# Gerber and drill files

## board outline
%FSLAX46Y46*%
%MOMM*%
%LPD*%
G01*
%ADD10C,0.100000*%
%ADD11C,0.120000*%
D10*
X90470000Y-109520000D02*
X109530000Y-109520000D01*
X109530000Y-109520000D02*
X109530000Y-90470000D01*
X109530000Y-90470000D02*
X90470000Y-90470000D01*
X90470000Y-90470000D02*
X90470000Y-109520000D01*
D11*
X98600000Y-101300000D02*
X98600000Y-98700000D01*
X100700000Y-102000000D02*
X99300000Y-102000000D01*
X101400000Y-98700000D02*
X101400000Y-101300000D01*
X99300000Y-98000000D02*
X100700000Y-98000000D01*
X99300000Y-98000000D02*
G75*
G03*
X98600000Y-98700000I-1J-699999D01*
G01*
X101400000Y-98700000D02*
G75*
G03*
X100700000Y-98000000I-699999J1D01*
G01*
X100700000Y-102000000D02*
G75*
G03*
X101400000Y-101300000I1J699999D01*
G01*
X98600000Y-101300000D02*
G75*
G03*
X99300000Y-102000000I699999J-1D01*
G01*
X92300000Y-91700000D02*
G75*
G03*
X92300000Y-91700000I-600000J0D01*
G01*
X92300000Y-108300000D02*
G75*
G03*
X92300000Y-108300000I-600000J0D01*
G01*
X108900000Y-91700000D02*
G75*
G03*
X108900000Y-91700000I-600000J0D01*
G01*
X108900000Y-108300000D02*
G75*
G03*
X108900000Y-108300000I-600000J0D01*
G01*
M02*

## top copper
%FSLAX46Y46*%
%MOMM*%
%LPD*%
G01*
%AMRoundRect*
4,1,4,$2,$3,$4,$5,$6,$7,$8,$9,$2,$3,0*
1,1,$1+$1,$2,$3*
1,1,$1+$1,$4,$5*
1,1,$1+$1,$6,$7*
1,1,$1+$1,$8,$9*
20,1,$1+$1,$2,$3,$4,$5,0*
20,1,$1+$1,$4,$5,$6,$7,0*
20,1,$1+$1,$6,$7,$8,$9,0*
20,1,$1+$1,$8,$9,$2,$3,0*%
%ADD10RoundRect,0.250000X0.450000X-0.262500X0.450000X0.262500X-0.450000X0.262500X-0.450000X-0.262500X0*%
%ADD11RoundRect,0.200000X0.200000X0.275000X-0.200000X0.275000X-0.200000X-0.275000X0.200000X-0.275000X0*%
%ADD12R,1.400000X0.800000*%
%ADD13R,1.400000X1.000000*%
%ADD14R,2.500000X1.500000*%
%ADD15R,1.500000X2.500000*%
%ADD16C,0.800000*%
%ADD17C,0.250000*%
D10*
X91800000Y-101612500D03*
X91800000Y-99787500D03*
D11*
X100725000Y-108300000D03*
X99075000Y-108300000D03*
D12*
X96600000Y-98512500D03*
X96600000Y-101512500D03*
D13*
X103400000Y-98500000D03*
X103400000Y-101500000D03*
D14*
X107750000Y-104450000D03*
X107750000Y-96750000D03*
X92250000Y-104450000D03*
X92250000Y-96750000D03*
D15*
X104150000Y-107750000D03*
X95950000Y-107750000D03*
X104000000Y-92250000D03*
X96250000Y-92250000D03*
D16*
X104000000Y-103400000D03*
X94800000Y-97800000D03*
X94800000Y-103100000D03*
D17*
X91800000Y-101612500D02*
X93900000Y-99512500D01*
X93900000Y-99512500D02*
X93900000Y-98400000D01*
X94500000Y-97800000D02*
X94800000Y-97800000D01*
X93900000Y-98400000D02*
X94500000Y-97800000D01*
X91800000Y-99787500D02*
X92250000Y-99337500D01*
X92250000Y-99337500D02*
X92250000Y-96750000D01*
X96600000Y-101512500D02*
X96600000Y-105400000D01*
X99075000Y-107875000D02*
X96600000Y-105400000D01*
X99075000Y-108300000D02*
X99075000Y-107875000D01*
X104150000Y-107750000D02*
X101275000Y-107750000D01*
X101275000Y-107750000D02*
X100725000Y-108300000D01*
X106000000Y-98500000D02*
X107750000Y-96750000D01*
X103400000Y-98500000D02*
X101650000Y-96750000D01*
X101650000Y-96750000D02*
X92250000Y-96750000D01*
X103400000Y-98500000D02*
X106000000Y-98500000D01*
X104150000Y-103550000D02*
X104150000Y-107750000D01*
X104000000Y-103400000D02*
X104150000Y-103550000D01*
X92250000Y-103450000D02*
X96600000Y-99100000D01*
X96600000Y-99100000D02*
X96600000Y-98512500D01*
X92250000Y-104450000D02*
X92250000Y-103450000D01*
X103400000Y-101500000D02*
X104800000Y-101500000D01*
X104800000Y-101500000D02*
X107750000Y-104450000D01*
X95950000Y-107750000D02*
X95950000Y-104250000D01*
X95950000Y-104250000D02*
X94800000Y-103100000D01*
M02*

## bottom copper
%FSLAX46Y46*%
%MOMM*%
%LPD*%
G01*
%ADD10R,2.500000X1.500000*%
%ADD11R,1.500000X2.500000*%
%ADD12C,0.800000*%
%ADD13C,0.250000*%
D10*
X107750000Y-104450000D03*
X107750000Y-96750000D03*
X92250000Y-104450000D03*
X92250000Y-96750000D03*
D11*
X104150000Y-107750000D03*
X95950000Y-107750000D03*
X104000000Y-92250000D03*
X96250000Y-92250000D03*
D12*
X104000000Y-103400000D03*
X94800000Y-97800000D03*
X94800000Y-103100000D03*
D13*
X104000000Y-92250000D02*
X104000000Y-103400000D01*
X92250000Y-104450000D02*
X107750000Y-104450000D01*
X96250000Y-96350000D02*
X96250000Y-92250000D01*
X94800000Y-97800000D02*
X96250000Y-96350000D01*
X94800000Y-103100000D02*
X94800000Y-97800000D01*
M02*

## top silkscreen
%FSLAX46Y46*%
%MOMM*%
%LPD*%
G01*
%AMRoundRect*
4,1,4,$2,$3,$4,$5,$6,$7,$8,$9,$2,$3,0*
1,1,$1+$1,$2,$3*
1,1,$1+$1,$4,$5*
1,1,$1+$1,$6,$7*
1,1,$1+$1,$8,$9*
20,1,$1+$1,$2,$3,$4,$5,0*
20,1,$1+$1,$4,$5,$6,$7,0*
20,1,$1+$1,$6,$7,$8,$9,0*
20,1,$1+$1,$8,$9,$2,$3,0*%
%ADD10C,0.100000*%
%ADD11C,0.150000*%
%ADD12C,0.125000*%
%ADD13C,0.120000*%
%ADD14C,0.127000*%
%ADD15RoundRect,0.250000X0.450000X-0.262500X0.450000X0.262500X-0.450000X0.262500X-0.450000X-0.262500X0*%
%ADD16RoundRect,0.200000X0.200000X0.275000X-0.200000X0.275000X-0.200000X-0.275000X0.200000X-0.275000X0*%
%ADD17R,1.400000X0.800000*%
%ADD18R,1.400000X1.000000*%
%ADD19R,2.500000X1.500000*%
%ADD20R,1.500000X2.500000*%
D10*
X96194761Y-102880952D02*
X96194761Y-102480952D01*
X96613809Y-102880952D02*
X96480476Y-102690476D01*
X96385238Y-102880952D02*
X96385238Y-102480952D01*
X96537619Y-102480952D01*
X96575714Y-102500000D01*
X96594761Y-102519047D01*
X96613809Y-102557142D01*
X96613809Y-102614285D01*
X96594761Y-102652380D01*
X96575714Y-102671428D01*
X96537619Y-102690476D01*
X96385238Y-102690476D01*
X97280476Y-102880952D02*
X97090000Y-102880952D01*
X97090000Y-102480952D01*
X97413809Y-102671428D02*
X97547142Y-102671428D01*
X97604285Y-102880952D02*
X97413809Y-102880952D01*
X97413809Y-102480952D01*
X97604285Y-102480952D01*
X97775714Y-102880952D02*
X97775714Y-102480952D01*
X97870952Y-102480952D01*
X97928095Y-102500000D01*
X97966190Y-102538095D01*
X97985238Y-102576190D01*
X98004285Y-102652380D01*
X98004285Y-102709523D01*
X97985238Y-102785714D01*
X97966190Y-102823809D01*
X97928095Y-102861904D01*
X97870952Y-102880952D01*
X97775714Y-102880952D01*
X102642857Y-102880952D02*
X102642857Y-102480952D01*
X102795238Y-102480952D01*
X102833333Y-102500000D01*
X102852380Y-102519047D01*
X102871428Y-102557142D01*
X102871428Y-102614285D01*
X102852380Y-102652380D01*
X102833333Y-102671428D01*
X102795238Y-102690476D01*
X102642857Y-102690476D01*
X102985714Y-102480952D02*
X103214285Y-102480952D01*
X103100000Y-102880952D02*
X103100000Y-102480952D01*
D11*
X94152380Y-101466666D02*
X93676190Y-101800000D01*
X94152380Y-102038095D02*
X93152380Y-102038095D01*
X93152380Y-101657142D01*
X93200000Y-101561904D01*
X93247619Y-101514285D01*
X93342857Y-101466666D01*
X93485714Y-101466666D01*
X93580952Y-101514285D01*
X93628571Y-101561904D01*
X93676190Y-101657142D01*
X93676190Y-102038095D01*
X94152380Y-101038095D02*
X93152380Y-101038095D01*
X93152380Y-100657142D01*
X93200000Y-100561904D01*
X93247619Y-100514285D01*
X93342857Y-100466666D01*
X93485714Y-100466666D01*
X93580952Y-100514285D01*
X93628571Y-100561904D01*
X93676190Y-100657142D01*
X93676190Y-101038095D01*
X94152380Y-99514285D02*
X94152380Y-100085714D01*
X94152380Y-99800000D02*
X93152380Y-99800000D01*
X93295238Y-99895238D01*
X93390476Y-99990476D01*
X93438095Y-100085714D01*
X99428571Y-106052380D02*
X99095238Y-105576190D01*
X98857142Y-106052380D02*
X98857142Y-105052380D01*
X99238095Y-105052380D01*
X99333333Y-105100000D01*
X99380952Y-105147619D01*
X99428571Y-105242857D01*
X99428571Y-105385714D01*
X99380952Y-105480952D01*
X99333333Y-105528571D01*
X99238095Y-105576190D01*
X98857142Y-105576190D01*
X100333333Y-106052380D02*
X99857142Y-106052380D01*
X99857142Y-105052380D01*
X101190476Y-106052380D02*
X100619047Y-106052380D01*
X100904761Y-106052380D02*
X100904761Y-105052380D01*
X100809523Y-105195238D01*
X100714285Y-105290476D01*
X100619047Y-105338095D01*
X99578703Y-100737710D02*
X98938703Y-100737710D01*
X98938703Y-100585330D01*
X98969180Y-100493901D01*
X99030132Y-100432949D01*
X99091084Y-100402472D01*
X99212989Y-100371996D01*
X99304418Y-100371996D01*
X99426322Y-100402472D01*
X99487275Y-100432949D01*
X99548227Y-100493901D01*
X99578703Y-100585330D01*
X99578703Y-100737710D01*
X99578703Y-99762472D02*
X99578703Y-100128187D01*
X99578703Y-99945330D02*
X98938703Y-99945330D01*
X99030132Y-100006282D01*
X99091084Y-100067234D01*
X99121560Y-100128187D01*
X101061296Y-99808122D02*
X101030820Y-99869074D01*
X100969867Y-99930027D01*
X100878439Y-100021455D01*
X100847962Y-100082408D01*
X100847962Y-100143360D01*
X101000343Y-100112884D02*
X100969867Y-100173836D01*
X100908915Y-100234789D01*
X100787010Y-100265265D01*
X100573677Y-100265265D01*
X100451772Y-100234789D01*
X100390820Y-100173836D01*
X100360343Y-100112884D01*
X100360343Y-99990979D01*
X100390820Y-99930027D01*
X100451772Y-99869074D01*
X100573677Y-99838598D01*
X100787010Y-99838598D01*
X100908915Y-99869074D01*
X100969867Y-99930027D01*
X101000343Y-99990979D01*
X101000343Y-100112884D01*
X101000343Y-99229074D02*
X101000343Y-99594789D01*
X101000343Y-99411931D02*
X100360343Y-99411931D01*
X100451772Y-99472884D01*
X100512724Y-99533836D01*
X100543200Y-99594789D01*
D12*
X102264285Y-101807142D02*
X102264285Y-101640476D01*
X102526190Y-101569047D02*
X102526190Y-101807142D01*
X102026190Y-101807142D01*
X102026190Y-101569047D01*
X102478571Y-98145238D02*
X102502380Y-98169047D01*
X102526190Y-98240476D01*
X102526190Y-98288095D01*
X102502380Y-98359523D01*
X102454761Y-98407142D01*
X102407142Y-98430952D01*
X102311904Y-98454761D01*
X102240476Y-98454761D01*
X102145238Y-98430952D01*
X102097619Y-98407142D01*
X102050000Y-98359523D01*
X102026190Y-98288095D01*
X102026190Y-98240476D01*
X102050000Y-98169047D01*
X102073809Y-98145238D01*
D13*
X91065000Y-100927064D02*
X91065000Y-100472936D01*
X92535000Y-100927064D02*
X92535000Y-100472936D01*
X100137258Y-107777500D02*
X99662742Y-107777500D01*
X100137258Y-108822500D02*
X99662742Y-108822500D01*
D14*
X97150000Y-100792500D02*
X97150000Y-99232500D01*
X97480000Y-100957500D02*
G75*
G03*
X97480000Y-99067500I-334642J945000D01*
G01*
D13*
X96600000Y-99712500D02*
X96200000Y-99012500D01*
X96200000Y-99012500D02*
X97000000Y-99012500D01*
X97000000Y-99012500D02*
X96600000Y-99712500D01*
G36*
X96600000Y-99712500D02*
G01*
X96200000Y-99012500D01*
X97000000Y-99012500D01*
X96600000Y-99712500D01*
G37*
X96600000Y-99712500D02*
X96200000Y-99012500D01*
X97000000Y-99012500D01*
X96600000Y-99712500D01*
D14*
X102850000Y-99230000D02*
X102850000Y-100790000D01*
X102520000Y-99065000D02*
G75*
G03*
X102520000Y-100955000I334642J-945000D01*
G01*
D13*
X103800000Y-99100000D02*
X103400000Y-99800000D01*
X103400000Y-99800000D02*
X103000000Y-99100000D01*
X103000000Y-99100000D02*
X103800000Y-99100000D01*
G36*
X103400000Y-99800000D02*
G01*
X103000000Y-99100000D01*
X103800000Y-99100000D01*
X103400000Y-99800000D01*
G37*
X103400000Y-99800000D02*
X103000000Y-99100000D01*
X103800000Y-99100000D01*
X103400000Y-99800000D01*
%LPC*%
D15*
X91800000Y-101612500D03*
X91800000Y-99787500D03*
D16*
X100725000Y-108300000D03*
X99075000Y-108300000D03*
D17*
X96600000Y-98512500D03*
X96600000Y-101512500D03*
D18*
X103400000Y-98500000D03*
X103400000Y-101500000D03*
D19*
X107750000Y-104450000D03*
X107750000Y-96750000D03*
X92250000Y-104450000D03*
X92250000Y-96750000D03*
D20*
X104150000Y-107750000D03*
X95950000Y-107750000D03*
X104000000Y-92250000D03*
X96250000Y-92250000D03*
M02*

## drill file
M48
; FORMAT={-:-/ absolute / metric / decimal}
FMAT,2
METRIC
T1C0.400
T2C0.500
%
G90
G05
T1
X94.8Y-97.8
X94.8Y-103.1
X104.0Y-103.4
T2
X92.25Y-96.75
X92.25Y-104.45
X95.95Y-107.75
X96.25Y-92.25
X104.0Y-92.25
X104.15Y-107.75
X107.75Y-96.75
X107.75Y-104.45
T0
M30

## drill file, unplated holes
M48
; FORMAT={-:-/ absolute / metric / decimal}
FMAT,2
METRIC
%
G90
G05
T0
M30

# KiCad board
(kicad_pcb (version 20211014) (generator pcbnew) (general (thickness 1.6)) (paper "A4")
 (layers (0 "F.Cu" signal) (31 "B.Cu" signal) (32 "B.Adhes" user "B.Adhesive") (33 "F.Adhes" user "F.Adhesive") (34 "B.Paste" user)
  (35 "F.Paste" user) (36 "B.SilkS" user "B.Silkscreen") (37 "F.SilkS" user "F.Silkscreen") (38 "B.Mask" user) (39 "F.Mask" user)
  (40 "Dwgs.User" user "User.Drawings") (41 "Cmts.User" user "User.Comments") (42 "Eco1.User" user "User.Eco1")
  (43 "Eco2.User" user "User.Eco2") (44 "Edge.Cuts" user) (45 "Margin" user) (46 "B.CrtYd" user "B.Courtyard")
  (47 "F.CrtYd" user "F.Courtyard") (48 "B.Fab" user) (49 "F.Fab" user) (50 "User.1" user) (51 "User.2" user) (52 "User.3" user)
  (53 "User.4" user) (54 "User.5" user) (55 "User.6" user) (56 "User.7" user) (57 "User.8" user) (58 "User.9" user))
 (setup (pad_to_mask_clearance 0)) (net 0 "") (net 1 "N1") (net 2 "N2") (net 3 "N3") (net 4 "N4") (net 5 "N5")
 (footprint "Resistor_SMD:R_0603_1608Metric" (layer "F.Cu") (at 99.9 108.3 180)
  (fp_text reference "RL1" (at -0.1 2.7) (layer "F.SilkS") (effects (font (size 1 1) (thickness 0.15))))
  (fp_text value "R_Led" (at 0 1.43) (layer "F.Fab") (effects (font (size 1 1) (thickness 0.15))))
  (fp_line (start -0.237258 -0.5225) (end 0.237258 -0.5225) (layer "F.SilkS") (width 0.12))
  (fp_line (start -0.237258 0.5225) (end 0.237258 0.5225) (layer "F.SilkS") (width 0.12))
  (pad "1" smd roundrect (at -0.825 0 180) (size 0.8 0.95) (layers "F.Cu" "F.Paste" "F.Mask") (roundrect_rratio 0.25) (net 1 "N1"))
  (pad "2" smd roundrect (at 0.825 0 180) (size 0.8 0.95) (layers "F.Cu" "F.Paste" "F.Mask") (roundrect_rratio 0.25) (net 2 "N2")))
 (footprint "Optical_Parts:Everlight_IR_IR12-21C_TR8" (layer "F.Cu") (at 96.6 100.0125 -90)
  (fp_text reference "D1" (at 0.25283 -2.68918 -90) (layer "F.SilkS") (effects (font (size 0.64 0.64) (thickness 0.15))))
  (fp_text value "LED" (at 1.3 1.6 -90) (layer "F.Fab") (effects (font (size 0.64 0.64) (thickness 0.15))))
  (fp_line (start 0.78 -0.55) (end -0.78 -0.55) (layer "F.SilkS") (width 0.127))
  (fp_arc (start -0.945 -0.88) (mid 0 -1.54786) (end 0.945 -0.88) (layer "F.SilkS") (width 0.127))
  (fp_poly (pts (xy -0.3 0) (xy -1 0.4) (xy -1 -0.4)) (layer "F.SilkS") (width 0.12) (fill solid))
  (pad "1" smd rect (at -1.5 0 270) (size 0.8 1.4) (layers "F.Cu" "F.Paste" "F.Mask") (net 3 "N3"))
  (pad "2" smd rect (at 1.5 0 270) (size 0.8 1.4) (layers "F.Cu" "F.Paste" "F.Mask") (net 2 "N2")))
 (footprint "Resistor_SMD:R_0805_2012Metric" (layer "F.Cu") (at 91.8 100.7 90)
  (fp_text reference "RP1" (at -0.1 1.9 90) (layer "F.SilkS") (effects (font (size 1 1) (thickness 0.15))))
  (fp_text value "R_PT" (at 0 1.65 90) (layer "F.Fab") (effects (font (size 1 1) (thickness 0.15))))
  (fp_line (start -0.227064 0.735) (end 0.227064 0.735) (layer "F.SilkS") (width 0.12))
  (fp_line (start -0.227064 -0.735) (end 0.227064 -0.735) (layer "F.SilkS") (width 0.12))
  (pad "1" smd roundrect (at -0.9125 0 90) (size 1.025 1.4) (layers "F.Cu" "F.Paste" "F.Mask") (roundrect_rratio 0.243902439) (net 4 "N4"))
  (pad "2" smd roundrect (at 0.9125 0 90) (size 1.025 1.4) (layers "F.Cu" "F.Paste" "F.Mask") (roundrect_rratio 0.243902439) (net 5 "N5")))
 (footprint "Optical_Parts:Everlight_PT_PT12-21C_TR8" (layer "F.Cu") (at 103.4 100 90)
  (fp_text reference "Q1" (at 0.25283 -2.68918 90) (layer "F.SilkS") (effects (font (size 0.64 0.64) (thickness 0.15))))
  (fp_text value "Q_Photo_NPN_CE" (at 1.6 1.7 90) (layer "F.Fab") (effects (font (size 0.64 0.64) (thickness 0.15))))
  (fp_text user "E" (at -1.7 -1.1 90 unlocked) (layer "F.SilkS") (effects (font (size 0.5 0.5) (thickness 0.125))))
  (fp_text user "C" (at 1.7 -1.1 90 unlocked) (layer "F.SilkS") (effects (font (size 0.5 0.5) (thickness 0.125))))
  (fp_line (start 0.77 -0.55) (end -0.79 -0.55) (layer "F.SilkS") (width 0.127))
  (fp_arc (start -0.955 -0.88) (mid -0.01 -1.54786) (end 0.935 -0.88) (layer "F.SilkS") (width 0.127))
  (fp_poly (pts (xy 0.9 0.4) (xy 0.2 0) (xy 0.9 -0.4)) (layer "F.SilkS") (width 0.12) (fill solid))
  (pad "1" smd rect (at 1.5 0 90) (size 1 1.4) (layers "F.Cu" "F.Paste" "F.Mask") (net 5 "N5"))
  (pad "2" smd rect (at -1.5 0 90) (size 1 1.4) (layers "F.Cu" "F.Paste" "F.Mask") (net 3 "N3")))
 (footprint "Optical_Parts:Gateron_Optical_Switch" (layer "F.Cu") (at 100 100)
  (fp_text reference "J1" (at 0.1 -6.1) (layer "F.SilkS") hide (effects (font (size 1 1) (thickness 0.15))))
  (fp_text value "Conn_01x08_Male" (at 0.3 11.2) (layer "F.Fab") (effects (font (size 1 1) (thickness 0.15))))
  (fp_line (start -1.4 1.3) (end -1.4 -1.3) (layer "Edge.Cuts") (width 0.12))
  (fp_line (start 0.7 2) (end -0.7 2) (layer "Edge.Cuts") (width 0.12))
  (fp_line (start 1.4 -1.3) (end 1.4 1.3) (layer "Edge.Cuts") (width 0.12))
  (fp_line (start -0.7 -2) (end 0.7 -2) (layer "Edge.Cuts") (width 0.12))
  (fp_arc (start -1.4 -1.3) (mid -1.194975 -1.794975) (end -0.7 -2) (layer "Edge.Cuts") (width 0.12))
  (fp_arc (start 0.7 -2) (mid 1.194975 -1.794975) (end 1.4 -1.3) (layer "Edge.Cuts") (width 0.12))
  (fp_arc (start 1.4 1.3) (mid 1.194975 1.794975) (end 0.7 2) (layer "Edge.Cuts") (width 0.12))
  (fp_arc (start -0.7 2) (mid -1.194975 1.794975) (end -1.4 1.3) (layer "Edge.Cuts") (width 0.12))
  (fp_circle (center -8.3 -8.3) (end -7.7 -8.3) (layer "Edge.Cuts") (width 0.12) (fill none))
  (fp_circle (center -8.3 8.3) (end -7.7 8.3) (layer "Edge.Cuts") (width 0.12) (fill none))
  (fp_circle (center 8.3 -8.3) (end 8.9 -8.3) (layer "Edge.Cuts") (width 0.12) (fill none))
  (fp_circle (center 8.3 8.3) (end 8.9 8.3) (layer "Edge.Cuts") (width 0.12) (fill none))
  (pad "1" thru_hole rect (at 7.75 4.45) (size 2.5 1.5) (drill 0.5) (layers *.Cu *.Mask) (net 3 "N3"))
  (pad "2" thru_hole rect (at 7.75 -3.25) (size 2.5 1.5) (drill 0.5) (layers *.Cu *.Mask) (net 5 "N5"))
  (pad "3" thru_hole rect (at -7.75 4.45) (size 2.5 1.5) (drill 0.5) (layers *.Cu *.Mask) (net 3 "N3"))
  (pad "4" thru_hole rect (at -7.75 -3.25) (size 2.5 1.5) (drill 0.5) (layers *.Cu *.Mask) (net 5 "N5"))
  (pad "5" thru_hole rect (at 4.15 7.75) (size 1.5 2.5) (drill 0.5) (layers *.Cu *.Mask) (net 1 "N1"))
  (pad "6" thru_hole rect (at -4.05 7.75) (size 1.5 2.5) (drill 0.5) (layers *.Cu *.Mask) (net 4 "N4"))
  (pad "7" thru_hole rect (at 4 -7.75) (size 1.5 2.5) (drill 0.5) (layers *.Cu *.Mask) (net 1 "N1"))
  (pad "8" thru_hole rect (at -3.75 -7.75) (size 1.5 2.5) (drill 0.5) (layers *.Cu *.Mask) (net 4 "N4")))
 (gr_rect (start 90.47 109.52) (end 109.53 90.47) (layer "Edge.Cuts") (width 0.1) (fill none))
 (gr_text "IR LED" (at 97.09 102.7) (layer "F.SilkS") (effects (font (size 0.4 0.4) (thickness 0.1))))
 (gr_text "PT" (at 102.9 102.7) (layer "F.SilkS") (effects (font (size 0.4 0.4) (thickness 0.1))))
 (segment (start 91.8 99.7875) (end 92.25 99.3375) (width 0.25) (layer "F.Cu") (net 5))
 (segment (start 106 98.5) (end 107.75 96.75) (width 0.25) (layer "F.Cu") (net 5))
 (segment (start 103.4 98.5) (end 101.65 96.75) (width 0.25) (layer "F.Cu") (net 5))
 (segment (start 101.65 96.75) (end 92.25 96.75) (width 0.25) (layer "F.Cu") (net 5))
 (segment (start 92.25 99.3375) (end 92.25 96.75) (width 0.25) (layer "F.Cu") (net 5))
 (segment (start 103.4 98.5) (end 106 98.5) (width 0.25) (layer "F.Cu") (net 5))
 (segment (start 104.15 103.55) (end 104.15 107.75) (width 0.25) (layer "F.Cu") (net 1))
 (segment (start 101.275 107.75) (end 100.725 108.3) (width 0.25) (layer "F.Cu") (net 1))
 (segment (start 104.15 107.75) (end 101.275 107.75) (width 0.25) (layer "F.Cu") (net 1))
 (segment (start 104 103.4) (end 104.15 103.55) (width 0.25) (layer "F.Cu") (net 1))
 (via (at 104 103.4) (size 0.8) (drill 0.4) (layers "F.Cu" "B.Cu") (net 1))
 (segment (start 104 92.25) (end 104 103.4) (width 0.25) (layer "B.Cu") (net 1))
 (segment (start 92.25 103.45) (end 96.6 99.1) (width 0.25) (layer "F.Cu") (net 3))
 (segment (start 96.6 99.1) (end 96.6 98.5125) (width 0.25) (layer "F.Cu") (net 3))
 (segment (start 92.25 104.45) (end 92.25 103.45) (width 0.25) (layer "F.Cu") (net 3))
 (segment (start 103.4 101.5) (end 104.8 101.5) (width 0.25) (layer "F.Cu") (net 3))
 (segment (start 104.8 101.5) (end 107.75 104.45) (width 0.25) (layer "F.Cu") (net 3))
 (segment (start 92.25 104.45) (end 107.75 104.45) (width 0.25) (layer "B.Cu") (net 3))
 (segment (start 96.6 101.5125) (end 96.6 105.4) (width 0.25) (layer "F.Cu") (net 2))
 (segment (start 99.075 108.3) (end 99.075 107.875) (width 0.25) (layer "F.Cu") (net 2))
 (segment (start 99.075 107.875) (end 96.6 105.4) (width 0.25) (layer "F.Cu") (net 2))
 (segment (start 95.95 107.75) (end 95.95 104.25) (width 0.25) (layer "F.Cu") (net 4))
 (segment (start 93.9 98.4) (end 94.5 97.8) (width 0.25) (layer "F.Cu") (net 4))
 (segment (start 95.95 104.25) (end 94.8 103.1) (width 0.25) (layer "F.Cu") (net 4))
 (segment (start 94.5 97.8) (end 94.8 97.8) (width 0.25) (layer "F.Cu") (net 4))
 (segment (start 93.9 99.5125) (end 93.9 98.4) (width 0.25) (layer "F.Cu") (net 4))
 (segment (start 91.8 101.6125) (end 93.9 99.5125) (width 0.25) (layer "F.Cu") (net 4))
 (via (at 94.8 97.8) (size 0.8) (drill 0.4) (layers "F.Cu" "B.Cu") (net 4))
 (via (at 94.8 103.1) (size 0.8) (drill 0.4) (layers "F.Cu" "B.Cu") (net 4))
 (segment (start 96.25 96.35) (end 96.25 92.25) (width 0.25) (layer "B.Cu") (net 4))
 (segment (start 94.8 97.8) (end 96.25 96.35) (width 0.25) (layer "B.Cu") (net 4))
 (segment (start 94.8 103.1) (end 94.8 97.8) (width 0.25) (layer "B.Cu") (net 4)))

